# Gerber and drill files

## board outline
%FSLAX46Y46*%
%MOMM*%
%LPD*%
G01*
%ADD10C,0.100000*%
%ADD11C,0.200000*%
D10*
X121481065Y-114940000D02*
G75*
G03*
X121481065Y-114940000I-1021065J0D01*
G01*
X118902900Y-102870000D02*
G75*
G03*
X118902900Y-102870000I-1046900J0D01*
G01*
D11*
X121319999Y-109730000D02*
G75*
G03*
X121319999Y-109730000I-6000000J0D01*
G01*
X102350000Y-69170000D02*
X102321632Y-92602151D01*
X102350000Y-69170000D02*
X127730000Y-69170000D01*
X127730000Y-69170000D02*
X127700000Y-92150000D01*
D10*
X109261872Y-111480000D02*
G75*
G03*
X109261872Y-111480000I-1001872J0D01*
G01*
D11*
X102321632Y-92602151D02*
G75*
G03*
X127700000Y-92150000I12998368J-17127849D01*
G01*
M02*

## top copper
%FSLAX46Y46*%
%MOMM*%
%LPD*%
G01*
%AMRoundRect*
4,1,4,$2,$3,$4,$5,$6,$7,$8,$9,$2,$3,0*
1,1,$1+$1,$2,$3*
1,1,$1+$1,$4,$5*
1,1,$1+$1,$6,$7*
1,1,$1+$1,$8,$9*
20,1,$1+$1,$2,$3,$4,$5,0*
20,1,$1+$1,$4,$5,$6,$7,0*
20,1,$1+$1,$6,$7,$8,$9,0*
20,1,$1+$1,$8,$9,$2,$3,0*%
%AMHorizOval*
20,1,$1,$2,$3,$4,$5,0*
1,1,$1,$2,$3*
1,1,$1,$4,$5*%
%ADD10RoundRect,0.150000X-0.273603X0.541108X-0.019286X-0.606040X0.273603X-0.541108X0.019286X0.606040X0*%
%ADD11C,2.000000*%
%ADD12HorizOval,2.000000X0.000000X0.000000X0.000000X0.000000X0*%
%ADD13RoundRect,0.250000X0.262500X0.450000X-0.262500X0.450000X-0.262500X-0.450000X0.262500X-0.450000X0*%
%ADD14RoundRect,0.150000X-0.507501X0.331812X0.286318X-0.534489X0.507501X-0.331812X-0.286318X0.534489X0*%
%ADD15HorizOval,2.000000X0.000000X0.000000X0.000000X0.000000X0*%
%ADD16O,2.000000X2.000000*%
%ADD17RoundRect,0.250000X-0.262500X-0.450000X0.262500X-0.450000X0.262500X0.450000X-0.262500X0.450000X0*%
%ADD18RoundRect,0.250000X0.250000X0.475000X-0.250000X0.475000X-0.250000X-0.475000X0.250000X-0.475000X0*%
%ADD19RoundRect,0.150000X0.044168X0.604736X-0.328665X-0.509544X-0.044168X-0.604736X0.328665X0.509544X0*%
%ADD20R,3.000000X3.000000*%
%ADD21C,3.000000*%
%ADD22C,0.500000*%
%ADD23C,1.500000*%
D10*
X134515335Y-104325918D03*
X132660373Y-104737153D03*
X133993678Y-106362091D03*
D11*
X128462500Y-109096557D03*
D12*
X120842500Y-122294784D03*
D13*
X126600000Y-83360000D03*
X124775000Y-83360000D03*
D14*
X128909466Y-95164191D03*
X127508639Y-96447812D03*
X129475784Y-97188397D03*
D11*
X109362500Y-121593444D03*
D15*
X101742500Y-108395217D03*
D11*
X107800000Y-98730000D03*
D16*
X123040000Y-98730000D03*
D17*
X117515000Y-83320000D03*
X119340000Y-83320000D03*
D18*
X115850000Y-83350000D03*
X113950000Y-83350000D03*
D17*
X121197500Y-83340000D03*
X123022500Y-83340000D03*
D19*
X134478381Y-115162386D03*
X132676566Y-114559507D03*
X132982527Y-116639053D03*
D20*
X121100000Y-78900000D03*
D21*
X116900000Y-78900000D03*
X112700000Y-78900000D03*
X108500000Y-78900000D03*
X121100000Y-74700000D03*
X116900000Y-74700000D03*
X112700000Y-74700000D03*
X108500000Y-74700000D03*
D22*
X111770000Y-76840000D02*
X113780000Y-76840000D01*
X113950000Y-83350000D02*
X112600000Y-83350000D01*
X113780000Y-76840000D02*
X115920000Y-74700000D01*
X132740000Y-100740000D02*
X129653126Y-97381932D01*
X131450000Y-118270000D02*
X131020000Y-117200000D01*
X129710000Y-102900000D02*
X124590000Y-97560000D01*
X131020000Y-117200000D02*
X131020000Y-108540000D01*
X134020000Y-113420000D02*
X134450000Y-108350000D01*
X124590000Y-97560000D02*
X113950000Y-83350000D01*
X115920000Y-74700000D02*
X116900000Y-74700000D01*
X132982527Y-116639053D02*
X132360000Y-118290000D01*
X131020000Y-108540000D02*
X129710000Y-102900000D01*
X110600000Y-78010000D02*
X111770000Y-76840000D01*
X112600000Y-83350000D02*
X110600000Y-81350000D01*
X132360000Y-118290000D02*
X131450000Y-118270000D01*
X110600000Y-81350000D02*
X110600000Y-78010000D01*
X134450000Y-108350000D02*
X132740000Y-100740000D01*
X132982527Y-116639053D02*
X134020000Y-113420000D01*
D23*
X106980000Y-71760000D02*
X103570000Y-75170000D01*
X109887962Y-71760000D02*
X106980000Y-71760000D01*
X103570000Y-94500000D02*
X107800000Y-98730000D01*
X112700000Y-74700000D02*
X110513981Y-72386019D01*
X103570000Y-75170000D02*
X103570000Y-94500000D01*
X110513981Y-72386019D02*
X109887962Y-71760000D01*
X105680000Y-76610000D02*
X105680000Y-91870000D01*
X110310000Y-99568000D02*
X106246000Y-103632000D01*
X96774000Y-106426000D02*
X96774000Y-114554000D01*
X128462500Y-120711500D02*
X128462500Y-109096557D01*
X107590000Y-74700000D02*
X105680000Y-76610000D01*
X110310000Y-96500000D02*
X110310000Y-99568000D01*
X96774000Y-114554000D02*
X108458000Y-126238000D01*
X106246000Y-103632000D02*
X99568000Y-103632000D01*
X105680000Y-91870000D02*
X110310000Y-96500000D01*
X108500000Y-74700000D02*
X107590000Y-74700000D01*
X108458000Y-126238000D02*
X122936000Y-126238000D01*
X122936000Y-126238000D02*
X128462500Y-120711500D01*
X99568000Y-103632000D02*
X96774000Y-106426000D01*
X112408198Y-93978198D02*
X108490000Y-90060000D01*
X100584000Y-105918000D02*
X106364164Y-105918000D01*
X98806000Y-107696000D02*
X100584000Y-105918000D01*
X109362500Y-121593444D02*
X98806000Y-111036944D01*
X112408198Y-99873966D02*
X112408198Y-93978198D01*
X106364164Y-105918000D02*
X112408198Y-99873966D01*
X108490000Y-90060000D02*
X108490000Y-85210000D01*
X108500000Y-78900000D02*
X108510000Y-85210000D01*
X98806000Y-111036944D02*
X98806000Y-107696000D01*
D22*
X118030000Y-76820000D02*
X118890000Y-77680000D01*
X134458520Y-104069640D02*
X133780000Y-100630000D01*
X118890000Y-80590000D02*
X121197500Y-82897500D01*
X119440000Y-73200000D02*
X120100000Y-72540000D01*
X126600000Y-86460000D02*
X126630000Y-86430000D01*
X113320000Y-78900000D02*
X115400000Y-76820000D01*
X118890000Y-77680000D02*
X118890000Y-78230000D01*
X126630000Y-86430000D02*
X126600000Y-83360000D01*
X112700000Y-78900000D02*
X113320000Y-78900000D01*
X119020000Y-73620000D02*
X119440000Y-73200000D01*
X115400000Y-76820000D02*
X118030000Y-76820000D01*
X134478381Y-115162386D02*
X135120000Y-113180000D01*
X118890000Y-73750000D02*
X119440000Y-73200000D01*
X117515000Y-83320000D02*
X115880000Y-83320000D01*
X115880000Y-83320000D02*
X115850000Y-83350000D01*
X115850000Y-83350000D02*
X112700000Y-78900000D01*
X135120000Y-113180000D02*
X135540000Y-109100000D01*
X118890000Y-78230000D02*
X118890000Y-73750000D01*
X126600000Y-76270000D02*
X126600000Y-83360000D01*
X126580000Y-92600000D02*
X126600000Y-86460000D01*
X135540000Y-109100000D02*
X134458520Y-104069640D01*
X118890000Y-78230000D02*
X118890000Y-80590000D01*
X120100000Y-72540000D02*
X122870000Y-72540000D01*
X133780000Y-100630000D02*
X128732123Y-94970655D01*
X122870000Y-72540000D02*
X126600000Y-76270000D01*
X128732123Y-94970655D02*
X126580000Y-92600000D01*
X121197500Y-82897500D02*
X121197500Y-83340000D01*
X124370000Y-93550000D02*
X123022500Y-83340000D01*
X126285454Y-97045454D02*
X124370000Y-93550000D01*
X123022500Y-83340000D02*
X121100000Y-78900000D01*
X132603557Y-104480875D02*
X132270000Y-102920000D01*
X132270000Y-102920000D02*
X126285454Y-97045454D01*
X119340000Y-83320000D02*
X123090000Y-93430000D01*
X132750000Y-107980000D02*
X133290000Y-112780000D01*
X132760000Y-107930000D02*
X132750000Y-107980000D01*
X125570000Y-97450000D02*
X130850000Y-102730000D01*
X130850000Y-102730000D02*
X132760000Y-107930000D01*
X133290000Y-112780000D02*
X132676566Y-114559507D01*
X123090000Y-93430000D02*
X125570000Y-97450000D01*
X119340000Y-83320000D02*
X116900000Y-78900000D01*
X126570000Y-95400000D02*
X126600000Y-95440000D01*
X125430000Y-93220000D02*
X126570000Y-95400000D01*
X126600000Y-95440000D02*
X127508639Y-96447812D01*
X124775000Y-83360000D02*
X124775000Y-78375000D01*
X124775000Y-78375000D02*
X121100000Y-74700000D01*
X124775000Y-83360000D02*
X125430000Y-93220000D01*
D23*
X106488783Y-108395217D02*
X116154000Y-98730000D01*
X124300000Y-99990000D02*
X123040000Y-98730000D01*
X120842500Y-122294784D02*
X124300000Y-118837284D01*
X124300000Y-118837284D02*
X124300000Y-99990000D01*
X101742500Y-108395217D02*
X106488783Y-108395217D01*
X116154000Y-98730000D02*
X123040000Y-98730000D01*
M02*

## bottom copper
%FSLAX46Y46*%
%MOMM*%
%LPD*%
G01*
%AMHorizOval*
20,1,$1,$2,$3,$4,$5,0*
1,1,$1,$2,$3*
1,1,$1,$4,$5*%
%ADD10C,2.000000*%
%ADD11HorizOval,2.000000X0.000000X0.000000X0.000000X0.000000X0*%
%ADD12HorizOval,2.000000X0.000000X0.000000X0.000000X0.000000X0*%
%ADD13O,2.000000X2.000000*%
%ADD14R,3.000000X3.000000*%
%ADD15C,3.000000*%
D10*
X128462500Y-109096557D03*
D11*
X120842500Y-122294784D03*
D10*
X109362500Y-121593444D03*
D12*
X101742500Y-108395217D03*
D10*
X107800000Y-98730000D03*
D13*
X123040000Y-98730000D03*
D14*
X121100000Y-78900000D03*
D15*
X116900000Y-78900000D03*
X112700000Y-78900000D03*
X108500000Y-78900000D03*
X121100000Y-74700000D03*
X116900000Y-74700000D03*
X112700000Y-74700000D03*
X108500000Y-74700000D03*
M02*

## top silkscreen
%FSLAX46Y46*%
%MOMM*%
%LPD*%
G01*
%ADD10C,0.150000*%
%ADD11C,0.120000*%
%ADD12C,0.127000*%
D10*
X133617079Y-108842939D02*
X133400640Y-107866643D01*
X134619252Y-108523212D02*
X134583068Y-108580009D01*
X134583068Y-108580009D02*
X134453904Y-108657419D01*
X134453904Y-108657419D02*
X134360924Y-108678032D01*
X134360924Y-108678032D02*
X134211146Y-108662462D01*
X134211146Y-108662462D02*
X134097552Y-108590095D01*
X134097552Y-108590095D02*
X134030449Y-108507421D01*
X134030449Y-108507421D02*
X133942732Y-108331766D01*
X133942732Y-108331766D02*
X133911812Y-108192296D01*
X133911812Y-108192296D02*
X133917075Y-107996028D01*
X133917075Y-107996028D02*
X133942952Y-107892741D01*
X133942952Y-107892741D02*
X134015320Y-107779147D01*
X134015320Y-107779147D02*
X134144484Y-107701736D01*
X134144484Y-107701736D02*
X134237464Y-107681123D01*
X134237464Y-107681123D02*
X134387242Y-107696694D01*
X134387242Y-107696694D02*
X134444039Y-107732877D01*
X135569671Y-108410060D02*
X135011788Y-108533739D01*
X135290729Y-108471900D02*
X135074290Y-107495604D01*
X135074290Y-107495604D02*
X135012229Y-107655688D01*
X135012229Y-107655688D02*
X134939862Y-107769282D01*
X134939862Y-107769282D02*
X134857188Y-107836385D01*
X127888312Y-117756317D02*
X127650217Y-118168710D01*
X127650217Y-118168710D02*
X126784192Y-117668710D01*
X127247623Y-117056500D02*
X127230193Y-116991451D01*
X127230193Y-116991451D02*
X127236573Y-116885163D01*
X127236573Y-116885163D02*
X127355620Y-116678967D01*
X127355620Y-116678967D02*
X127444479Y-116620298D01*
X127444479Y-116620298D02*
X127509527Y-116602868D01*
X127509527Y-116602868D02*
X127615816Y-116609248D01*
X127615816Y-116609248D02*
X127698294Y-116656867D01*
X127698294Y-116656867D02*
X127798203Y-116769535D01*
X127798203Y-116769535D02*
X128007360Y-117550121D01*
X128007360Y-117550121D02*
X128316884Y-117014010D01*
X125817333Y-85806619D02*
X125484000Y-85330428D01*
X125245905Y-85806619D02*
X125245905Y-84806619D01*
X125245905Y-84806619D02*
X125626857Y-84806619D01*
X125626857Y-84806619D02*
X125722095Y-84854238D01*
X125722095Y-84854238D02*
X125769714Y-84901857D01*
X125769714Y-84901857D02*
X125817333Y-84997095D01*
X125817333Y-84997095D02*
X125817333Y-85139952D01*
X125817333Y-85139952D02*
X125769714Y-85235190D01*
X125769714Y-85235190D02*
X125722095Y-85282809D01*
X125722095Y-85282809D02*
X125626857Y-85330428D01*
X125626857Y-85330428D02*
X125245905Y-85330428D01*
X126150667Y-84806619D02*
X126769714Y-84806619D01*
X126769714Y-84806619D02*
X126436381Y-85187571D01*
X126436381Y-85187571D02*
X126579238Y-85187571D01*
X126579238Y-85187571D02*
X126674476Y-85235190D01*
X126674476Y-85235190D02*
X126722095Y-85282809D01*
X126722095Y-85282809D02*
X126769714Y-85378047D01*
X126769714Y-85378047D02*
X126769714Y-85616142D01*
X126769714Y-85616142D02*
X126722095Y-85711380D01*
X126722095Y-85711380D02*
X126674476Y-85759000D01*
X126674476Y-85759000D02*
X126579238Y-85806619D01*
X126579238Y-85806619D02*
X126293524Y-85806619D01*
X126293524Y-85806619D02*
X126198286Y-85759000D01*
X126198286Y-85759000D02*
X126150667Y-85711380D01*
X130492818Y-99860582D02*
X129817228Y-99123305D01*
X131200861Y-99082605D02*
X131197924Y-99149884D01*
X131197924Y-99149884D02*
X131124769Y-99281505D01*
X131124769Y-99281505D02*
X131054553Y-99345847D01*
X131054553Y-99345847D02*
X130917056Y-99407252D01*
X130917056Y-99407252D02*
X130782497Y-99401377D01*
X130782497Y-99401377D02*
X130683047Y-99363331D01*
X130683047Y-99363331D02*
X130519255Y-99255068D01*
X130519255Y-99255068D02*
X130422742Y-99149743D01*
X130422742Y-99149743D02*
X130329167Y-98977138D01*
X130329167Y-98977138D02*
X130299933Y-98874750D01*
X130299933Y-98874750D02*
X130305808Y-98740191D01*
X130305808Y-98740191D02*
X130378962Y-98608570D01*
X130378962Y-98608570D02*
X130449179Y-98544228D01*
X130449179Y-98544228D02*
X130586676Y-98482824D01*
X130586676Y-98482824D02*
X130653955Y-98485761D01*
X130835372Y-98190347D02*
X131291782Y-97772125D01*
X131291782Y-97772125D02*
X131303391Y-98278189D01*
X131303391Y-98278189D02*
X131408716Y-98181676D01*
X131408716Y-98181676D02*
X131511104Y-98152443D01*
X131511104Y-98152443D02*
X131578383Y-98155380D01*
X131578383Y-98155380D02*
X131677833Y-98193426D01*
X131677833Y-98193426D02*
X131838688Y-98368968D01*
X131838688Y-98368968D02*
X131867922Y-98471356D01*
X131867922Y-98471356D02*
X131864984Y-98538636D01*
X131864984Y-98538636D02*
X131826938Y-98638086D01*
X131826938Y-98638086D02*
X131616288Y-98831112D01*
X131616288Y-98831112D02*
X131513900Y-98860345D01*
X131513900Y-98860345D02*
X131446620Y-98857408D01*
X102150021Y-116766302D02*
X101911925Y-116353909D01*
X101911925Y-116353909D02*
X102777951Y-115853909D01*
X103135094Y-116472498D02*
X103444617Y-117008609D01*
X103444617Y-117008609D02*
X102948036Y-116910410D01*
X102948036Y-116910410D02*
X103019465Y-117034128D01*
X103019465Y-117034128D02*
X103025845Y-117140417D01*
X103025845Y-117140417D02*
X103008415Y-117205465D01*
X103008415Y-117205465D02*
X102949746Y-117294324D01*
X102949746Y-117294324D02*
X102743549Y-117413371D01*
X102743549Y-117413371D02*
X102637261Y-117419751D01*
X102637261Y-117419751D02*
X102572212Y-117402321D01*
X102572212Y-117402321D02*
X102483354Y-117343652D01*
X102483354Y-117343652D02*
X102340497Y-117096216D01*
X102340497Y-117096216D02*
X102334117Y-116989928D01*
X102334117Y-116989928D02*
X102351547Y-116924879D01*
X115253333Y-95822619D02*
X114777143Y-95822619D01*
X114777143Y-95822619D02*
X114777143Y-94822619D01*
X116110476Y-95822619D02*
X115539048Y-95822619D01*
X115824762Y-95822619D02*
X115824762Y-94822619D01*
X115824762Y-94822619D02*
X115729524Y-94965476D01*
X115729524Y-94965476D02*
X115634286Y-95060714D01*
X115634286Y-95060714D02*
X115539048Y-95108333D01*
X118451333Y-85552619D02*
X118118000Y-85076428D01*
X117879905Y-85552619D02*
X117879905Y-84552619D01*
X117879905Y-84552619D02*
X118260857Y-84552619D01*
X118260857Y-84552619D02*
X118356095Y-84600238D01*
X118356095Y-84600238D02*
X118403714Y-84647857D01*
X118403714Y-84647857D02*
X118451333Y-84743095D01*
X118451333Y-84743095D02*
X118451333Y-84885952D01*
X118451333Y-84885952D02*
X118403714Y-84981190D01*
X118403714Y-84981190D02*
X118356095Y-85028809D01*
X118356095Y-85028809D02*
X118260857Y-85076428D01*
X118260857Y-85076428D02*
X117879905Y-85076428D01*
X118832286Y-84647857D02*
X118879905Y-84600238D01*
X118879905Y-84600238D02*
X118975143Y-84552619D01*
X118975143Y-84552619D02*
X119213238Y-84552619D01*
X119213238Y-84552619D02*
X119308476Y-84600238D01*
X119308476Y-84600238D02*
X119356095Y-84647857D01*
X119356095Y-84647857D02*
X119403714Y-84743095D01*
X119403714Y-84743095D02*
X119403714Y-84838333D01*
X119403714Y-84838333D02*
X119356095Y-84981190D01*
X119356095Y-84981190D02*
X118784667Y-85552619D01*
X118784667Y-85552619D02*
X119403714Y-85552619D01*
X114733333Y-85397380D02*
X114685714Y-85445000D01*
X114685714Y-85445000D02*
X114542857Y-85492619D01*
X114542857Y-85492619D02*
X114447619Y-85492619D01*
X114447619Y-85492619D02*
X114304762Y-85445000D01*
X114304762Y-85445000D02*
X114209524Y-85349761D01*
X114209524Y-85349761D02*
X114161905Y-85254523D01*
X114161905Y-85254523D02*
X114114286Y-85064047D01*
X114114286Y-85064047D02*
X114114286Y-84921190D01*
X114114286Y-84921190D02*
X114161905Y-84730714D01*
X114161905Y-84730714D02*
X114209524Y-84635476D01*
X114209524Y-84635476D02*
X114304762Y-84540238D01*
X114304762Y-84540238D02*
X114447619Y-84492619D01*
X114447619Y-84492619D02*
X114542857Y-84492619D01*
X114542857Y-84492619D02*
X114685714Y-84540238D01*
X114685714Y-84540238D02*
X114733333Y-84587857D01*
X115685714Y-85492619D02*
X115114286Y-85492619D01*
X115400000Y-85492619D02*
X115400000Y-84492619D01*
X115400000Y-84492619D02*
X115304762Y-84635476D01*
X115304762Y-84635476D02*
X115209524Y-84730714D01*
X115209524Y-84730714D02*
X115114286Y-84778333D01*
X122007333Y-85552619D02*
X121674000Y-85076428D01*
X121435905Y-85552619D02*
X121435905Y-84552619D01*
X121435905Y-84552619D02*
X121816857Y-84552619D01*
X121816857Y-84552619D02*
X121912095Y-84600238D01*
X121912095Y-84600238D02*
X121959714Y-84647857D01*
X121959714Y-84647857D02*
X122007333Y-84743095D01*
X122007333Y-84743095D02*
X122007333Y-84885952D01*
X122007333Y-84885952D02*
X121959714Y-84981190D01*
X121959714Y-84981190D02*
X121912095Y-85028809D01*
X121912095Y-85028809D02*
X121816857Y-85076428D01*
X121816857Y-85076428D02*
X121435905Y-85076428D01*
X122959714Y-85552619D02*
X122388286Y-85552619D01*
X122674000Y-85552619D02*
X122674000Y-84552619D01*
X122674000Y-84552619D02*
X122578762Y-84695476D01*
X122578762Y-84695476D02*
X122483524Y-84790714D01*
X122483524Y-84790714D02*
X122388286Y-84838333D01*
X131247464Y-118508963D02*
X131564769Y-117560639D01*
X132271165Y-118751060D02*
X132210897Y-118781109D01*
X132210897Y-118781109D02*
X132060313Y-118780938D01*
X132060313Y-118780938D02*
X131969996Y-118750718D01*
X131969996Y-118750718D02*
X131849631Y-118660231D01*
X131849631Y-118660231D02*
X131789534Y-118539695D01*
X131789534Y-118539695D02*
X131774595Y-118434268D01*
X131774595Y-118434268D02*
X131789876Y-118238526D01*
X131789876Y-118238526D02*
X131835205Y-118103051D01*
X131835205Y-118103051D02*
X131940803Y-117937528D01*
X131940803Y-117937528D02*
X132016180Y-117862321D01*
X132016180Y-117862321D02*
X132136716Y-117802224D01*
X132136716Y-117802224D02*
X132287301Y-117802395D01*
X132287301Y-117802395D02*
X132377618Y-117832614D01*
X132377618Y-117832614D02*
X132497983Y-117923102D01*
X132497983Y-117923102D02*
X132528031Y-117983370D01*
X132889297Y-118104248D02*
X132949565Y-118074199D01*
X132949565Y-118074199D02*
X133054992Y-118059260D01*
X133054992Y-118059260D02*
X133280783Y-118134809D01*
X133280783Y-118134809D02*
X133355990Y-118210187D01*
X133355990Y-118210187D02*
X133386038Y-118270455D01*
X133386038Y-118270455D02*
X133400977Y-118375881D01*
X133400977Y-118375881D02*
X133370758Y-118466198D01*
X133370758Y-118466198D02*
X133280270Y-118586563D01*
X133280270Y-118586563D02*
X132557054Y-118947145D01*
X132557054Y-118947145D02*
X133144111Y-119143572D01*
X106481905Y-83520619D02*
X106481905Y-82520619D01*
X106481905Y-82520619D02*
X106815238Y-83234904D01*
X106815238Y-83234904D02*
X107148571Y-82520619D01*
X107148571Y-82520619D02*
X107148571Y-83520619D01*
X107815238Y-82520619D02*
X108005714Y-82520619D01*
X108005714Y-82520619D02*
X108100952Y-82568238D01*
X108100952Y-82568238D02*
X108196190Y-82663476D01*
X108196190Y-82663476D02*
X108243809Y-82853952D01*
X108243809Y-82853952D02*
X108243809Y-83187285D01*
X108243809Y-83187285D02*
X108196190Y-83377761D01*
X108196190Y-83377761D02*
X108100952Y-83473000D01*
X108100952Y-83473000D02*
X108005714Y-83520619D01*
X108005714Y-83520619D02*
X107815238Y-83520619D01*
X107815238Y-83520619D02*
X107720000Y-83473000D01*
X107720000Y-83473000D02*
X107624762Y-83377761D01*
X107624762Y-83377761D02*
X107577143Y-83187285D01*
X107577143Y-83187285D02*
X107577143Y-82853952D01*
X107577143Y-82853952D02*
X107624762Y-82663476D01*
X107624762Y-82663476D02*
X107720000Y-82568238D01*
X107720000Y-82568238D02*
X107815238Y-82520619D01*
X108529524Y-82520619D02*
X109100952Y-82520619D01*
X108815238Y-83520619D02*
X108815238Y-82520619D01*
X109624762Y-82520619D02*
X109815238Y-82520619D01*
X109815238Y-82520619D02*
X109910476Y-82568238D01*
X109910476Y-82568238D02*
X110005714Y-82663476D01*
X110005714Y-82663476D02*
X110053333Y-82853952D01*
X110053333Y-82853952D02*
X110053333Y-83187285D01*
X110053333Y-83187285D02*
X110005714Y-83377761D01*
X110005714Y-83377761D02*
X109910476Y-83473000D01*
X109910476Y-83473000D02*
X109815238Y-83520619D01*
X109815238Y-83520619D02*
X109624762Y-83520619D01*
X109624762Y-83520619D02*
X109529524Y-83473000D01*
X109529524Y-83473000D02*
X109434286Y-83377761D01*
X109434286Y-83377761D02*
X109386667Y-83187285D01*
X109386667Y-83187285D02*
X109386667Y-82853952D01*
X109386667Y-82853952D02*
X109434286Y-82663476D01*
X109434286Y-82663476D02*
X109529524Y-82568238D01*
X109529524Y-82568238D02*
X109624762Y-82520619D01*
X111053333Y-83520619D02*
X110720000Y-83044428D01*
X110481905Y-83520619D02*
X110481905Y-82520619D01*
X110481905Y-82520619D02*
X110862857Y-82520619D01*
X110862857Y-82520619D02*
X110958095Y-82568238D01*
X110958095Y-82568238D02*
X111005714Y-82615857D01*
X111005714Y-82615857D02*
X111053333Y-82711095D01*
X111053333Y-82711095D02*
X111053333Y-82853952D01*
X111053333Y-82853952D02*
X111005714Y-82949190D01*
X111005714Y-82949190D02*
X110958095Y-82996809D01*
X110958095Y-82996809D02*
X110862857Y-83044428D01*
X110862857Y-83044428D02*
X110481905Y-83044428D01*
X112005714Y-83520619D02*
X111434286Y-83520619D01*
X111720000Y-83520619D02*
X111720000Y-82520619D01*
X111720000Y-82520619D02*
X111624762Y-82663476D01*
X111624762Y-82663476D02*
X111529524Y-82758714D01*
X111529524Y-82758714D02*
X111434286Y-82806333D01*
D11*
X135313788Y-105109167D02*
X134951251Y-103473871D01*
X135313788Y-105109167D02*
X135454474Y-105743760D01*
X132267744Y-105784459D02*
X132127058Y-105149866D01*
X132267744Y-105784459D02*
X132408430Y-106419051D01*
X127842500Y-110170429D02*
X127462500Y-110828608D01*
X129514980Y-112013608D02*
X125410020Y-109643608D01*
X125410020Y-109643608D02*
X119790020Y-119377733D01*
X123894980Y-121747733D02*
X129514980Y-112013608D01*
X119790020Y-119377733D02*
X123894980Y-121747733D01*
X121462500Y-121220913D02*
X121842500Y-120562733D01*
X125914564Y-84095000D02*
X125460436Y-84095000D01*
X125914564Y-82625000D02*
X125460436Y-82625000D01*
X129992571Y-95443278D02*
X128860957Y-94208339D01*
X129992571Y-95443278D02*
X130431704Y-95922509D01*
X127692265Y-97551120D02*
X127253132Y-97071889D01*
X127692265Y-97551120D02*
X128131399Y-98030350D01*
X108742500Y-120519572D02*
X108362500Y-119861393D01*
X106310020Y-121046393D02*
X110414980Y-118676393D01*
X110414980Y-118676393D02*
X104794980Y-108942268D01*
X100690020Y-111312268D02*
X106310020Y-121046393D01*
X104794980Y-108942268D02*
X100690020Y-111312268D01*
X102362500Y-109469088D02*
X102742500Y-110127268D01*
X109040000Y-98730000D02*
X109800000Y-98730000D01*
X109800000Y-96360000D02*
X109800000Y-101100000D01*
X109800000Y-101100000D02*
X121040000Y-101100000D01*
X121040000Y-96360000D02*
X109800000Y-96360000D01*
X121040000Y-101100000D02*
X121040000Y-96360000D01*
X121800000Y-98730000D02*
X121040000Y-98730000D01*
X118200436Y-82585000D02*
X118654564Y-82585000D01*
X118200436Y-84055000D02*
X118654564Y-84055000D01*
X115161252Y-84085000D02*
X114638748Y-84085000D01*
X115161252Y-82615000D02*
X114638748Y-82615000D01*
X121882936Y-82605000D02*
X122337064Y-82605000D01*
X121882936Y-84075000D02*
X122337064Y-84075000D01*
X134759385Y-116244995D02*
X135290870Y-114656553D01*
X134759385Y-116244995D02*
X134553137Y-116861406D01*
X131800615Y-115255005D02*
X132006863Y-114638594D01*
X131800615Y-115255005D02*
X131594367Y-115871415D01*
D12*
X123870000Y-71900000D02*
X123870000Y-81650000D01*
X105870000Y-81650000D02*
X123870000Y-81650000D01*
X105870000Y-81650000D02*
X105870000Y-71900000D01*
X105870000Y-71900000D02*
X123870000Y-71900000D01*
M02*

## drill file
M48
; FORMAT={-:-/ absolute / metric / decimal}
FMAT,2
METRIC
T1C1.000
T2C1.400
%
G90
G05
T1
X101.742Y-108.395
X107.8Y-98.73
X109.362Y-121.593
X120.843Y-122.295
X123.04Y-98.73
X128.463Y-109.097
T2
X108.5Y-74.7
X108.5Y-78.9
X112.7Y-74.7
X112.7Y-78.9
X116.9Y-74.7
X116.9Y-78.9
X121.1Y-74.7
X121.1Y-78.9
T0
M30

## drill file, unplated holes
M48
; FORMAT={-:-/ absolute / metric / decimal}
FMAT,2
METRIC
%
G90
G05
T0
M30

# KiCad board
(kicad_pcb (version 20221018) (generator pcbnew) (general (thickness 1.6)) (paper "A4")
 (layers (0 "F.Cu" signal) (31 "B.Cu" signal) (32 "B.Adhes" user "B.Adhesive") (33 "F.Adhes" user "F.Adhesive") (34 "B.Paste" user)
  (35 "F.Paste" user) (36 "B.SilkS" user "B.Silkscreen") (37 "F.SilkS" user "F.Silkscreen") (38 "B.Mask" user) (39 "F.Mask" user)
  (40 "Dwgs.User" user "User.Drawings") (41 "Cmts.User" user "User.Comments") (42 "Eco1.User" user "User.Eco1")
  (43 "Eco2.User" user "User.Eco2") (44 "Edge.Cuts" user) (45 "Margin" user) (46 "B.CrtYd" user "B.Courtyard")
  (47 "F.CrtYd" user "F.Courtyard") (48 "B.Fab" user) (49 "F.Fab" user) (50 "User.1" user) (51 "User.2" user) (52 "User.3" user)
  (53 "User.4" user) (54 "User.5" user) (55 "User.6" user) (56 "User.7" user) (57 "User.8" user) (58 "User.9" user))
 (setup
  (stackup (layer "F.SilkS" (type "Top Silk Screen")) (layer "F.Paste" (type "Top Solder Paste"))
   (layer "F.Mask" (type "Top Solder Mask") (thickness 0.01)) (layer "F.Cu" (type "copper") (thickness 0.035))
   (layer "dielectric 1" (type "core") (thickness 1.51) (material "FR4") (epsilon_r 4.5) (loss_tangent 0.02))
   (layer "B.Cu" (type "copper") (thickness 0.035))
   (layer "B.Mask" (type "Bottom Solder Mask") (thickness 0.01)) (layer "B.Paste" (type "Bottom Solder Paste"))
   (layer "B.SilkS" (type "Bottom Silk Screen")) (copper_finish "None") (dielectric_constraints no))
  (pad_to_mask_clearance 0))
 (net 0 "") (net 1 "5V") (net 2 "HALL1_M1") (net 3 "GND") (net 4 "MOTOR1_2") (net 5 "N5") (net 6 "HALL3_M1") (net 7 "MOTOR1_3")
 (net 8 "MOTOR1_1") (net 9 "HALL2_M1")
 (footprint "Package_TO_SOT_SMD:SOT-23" (layer "F.Cu") (at 133.790766 105.446813 -77.5)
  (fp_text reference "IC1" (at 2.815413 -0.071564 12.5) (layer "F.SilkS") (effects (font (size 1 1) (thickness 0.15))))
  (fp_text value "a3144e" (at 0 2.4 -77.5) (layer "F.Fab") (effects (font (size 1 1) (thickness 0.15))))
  (fp_line (start 0 -1.56) (end -1.675 -1.56) (stroke (width 0.12) (type solid)) (layer "F.SilkS"))
  (fp_line (start 0 -1.56) (end 0.65 -1.56) (stroke (width 0.12) (type solid)) (layer "F.SilkS"))
  (fp_line (start 0 1.56) (end -0.65 1.56) (stroke (width 0.12) (type solid)) (layer "F.SilkS"))
  (fp_line (start 0 1.56) (end 0.65 1.56) (stroke (width 0.12) (type solid)) (layer "F.SilkS"))
  (pad "1" smd roundrect (at -0.9375 -0.95 282.5) (size 1.475 0.6) (layers "F.Cu" "F.Paste" "F.Mask") (roundrect_rratio 0.25) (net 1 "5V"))
  (pad "2" smd roundrect (at -0.9375 0.95 282.5) (size 1.475 0.6) (layers "F.Cu" "F.Paste" "F.Mask") (roundrect_rratio 0.25)
   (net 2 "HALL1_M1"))
  (pad "3" smd roundrect (at 0.9375 0 282.5) (size 1.475 0.6) (layers "F.Cu" "F.Paste" "F.Mask") (roundrect_rratio 0.25) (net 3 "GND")))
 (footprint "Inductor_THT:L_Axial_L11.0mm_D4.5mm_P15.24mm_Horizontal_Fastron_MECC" (layer "F.Cu") (at 128.4625 109.096557 -120)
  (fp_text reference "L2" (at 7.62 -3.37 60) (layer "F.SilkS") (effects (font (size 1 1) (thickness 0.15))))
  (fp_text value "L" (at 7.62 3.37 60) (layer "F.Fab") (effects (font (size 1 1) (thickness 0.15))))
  (fp_line (start 1.24 0) (end 2 0) (stroke (width 0.12) (type solid)) (layer "F.SilkS"))
  (fp_line (start 2 -2.37) (end 2 2.37) (stroke (width 0.12) (type solid)) (layer "F.SilkS"))
  (fp_line (start 2 2.37) (end 13.24 2.37) (stroke (width 0.12) (type solid)) (layer "F.SilkS"))
  (fp_line (start 13.24 -2.37) (end 2 -2.37) (stroke (width 0.12) (type solid)) (layer "F.SilkS"))
  (fp_line (start 13.24 2.37) (end 13.24 -2.37) (stroke (width 0.12) (type solid)) (layer "F.SilkS"))
  (fp_line (start 14 0) (end 13.24 0) (stroke (width 0.12) (type solid)) (layer "F.SilkS"))
  (pad "1" thru_hole circle (at 0 0 240) (size 2 2) (drill 1) (layers "*.Cu" "*.Mask") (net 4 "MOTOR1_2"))
  (pad "2" thru_hole oval (at 15.24 0 240) (size 2 2) (drill 1) (layers "*.Cu" "*.Mask") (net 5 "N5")))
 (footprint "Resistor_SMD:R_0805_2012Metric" (layer "F.Cu") (at 125.6875 83.36 180)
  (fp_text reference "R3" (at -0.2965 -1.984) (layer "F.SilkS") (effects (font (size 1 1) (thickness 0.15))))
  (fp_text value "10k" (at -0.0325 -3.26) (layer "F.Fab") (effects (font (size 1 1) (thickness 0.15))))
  (fp_line (start -0.227064 -0.735) (end 0.227064 -0.735) (stroke (width 0.12) (type solid)) (layer "F.SilkS"))
  (fp_line (start -0.227064 0.735) (end 0.227064 0.735) (stroke (width 0.12) (type solid)) (layer "F.SilkS"))
  (pad "1" smd roundrect (at -0.9125 0 180) (size 1.025 1.4) (layers "F.Cu" "F.Paste" "F.Mask") (roundrect_rratio 0.243902439) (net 1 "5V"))
  (pad "2" smd roundrect (at 0.9125 0 180) (size 1.025 1.4) (layers "F.Cu" "F.Paste" "F.Mask") (roundrect_rratio 0.243902439)
   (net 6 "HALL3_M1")))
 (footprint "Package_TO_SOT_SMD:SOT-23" (layer "F.Cu") (at 128.842418 96.497199 -47.5)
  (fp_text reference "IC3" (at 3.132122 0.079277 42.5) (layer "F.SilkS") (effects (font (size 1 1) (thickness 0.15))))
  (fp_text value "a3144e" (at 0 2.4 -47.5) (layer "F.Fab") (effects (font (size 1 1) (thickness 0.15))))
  (fp_line (start 0 -1.56) (end -1.675 -1.56) (stroke (width 0.12) (type solid)) (layer "F.SilkS"))
  (fp_line (start 0 -1.56) (end 0.65 -1.56) (stroke (width 0.12) (type solid)) (layer "F.SilkS"))
  (fp_line (start 0 1.56) (end -0.65 1.56) (stroke (width 0.12) (type solid)) (layer "F.SilkS"))
  (fp_line (start 0 1.56) (end 0.65 1.56) (stroke (width 0.12) (type solid)) (layer "F.SilkS"))
  (pad "1" smd roundrect (at -0.9375 -0.95 312.5) (size 1.475 0.6) (layers "F.Cu" "F.Paste" "F.Mask") (roundrect_rratio 0.25) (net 1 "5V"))
  (pad "2" smd roundrect (at -0.9375 0.95 312.5) (size 1.475 0.6) (layers "F.Cu" "F.Paste" "F.Mask") (roundrect_rratio 0.25)
   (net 6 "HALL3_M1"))
  (pad "3" smd roundrect (at 0.9375 0 312.5) (size 1.475 0.6) (layers "F.Cu" "F.Paste" "F.Mask") (roundrect_rratio 0.25) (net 3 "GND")))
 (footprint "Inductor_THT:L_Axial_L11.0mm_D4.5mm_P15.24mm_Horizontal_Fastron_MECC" (layer "F.Cu") (at 109.3625 121.593444 120)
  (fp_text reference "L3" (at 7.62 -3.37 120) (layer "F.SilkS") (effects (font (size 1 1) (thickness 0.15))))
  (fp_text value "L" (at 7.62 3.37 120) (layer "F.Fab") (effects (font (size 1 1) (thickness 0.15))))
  (fp_line (start 1.24 0) (end 2 0) (stroke (width 0.12) (type solid)) (layer "F.SilkS"))
  (fp_line (start 2 -2.37) (end 2 2.37) (stroke (width 0.12) (type solid)) (layer "F.SilkS"))
  (fp_line (start 2 2.37) (end 13.24 2.37) (stroke (width 0.12) (type solid)) (layer "F.SilkS"))
  (fp_line (start 13.24 -2.37) (end 2 -2.37) (stroke (width 0.12) (type solid)) (layer "F.SilkS"))
  (fp_line (start 13.24 2.37) (end 13.24 -2.37) (stroke (width 0.12) (type solid)) (layer "F.SilkS"))
  (fp_line (start 14 0) (end 13.24 0) (stroke (width 0.12) (type solid)) (layer "F.SilkS"))
  (pad "1" thru_hole circle (at 0 0 120) (size 2 2) (drill 1) (layers "*.Cu" "*.Mask") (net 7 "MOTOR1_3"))
  (pad "2" thru_hole oval (at 15.24 0 120) (size 2 2) (drill 1) (layers "*.Cu" "*.Mask") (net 5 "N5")))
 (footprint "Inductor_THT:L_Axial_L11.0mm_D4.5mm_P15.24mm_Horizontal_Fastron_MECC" (layer "F.Cu") (at 107.8 98.73)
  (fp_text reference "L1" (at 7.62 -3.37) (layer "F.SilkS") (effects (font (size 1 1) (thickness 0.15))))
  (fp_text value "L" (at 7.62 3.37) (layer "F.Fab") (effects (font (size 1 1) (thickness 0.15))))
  (fp_line (start 1.24 0) (end 2 0) (stroke (width 0.12) (type solid)) (layer "F.SilkS"))
  (fp_line (start 2 -2.37) (end 2 2.37) (stroke (width 0.12) (type solid)) (layer "F.SilkS"))
  (fp_line (start 2 2.37) (end 13.24 2.37) (stroke (width 0.12) (type solid)) (layer "F.SilkS"))
  (fp_line (start 13.24 -2.37) (end 2 -2.37) (stroke (width 0.12) (type solid)) (layer "F.SilkS"))
  (fp_line (start 13.24 2.37) (end 13.24 -2.37) (stroke (width 0.12) (type solid)) (layer "F.SilkS"))
  (fp_line (start 14 0) (end 13.24 0) (stroke (width 0.12) (type solid)) (layer "F.SilkS"))
  (pad "1" thru_hole circle (at 0 0) (size 2 2) (drill 1) (layers "*.Cu" "*.Mask") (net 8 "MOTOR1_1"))
  (pad "2" thru_hole oval (at 15.24 0) (size 2 2) (drill 1) (layers "*.Cu" "*.Mask") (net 5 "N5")))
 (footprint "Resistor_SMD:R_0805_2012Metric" (layer "F.Cu") (at 118.4275 83.32)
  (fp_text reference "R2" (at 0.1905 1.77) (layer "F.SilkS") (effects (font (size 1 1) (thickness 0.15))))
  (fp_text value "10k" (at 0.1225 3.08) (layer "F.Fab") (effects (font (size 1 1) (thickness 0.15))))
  (fp_line (start -0.227064 -0.735) (end 0.227064 -0.735) (stroke (width 0.12) (type solid)) (layer "F.SilkS"))
  (fp_line (start -0.227064 0.735) (end 0.227064 0.735) (stroke (width 0.12) (type solid)) (layer "F.SilkS"))
  (pad "1" smd roundrect (at -0.9125 0) (size 1.025 1.4) (layers "F.Cu" "F.Paste" "F.Mask") (roundrect_rratio 0.243902439) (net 1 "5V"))
  (pad "2" smd roundrect (at 0.9125 0) (size 1.025 1.4) (layers "F.Cu" "F.Paste" "F.Mask") (roundrect_rratio 0.243902439) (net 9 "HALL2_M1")))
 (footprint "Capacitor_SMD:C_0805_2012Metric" (layer "F.Cu") (at 114.9 83.35 180)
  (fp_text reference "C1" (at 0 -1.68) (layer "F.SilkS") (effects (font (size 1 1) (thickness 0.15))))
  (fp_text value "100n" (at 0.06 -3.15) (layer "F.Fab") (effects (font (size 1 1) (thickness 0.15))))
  (fp_line (start -0.261252 -0.735) (end 0.261252 -0.735) (stroke (width 0.12) (type solid)) (layer "F.SilkS"))
  (fp_line (start -0.261252 0.735) (end 0.261252 0.735) (stroke (width 0.12) (type solid)) (layer "F.SilkS"))
  (pad "1" smd roundrect (at -0.95 0 180) (size 1 1.45) (layers "F.Cu" "F.Paste" "F.Mask") (roundrect_rratio 0.25) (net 1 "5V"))
  (pad "2" smd roundrect (at 0.95 0 180) (size 1 1.45) (layers "F.Cu" "F.Paste" "F.Mask") (roundrect_rratio 0.25) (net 3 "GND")))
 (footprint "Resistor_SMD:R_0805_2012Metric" (layer "F.Cu") (at 122.11 83.34)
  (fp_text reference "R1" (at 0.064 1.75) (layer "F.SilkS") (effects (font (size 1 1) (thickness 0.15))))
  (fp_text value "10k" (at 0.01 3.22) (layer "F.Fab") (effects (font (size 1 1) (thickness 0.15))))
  (fp_line (start -0.227064 -0.735) (end 0.227064 -0.735) (stroke (width 0.12) (type solid)) (layer "F.SilkS"))
  (fp_line (start -0.227064 0.735) (end 0.227064 0.735) (stroke (width 0.12) (type solid)) (layer "F.SilkS"))
  (pad "1" smd roundrect (at -0.9125 0) (size 1.025 1.4) (layers "F.Cu" "F.Paste" "F.Mask") (roundrect_rratio 0.243902439) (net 1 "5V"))
  (pad "2" smd roundrect (at 0.9125 0) (size 1.025 1.4) (layers "F.Cu" "F.Paste" "F.Mask") (roundrect_rratio 0.243902439) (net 2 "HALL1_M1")))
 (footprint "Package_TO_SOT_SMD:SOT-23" (layer "F.Cu") (at 133.28 115.75 -108.5)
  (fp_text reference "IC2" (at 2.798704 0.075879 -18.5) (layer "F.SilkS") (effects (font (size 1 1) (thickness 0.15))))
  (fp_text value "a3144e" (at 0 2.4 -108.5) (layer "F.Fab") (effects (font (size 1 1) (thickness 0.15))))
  (fp_line (start 0 -1.56) (end -1.675 -1.56) (stroke (width 0.12) (type solid)) (layer "F.SilkS"))
  (fp_line (start 0 -1.56) (end 0.65 -1.56) (stroke (width 0.12) (type solid)) (layer "F.SilkS"))
  (fp_line (start 0 1.56) (end -0.65 1.56) (stroke (width 0.12) (type solid)) (layer "F.SilkS"))
  (fp_line (start 0 1.56) (end 0.65 1.56) (stroke (width 0.12) (type solid)) (layer "F.SilkS"))
  (pad "1" smd roundrect (at -0.9375 -0.95 251.5) (size 1.475 0.6) (layers "F.Cu" "F.Paste" "F.Mask") (roundrect_rratio 0.25) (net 1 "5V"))
  (pad "2" smd roundrect (at -0.9375 0.95 251.5) (size 1.475 0.6) (layers "F.Cu" "F.Paste" "F.Mask") (roundrect_rratio 0.25)
   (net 9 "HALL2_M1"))
  (pad "3" smd roundrect (at 0.9375 0 251.5) (size 1.475 0.6) (layers "F.Cu" "F.Paste" "F.Mask") (roundrect_rratio 0.25) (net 3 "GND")))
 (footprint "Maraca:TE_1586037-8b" (layer "F.Cu") (at 121.1 78.9 180)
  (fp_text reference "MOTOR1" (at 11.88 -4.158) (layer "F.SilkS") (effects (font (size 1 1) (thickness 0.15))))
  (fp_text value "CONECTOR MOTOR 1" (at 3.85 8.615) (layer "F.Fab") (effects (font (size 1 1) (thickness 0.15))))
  (fp_line (start -2.77 7) (end -2.77 -2.75) (stroke (width 0.127) (type solid)) (layer "F.SilkS"))
  (fp_line (start 15.23 -2.75) (end -2.77 -2.75) (stroke (width 0.127) (type solid)) (layer "F.SilkS"))
  (fp_line (start 15.23 -2.75) (end 15.23 7) (stroke (width 0.127) (type solid)) (layer "F.SilkS"))
  (fp_line (start 15.23 7) (end -2.77 7) (stroke (width 0.127) (type solid)) (layer "F.SilkS"))
  (pad "1" thru_hole rect (at 0 0 180) (size 3 3) (drill 1.4) (layers "*.Cu" "*.Mask") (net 2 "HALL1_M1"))
  (pad "2" thru_hole circle (at 4.2 0 180) (size 3 3) (drill 1.4) (layers "*.Cu" "*.Mask") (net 9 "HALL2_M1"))
  (pad "3" thru_hole circle (at 8.4 0 180) (size 3 3) (drill 1.4) (layers "*.Cu" "*.Mask") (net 1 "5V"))
  (pad "4" thru_hole circle (at 12.6 0 180) (size 3 3) (drill 1.4) (layers "*.Cu" "*.Mask") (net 7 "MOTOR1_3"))
  (pad "5" thru_hole circle (at 0 4.2 180) (size 3 3) (drill 1.4) (layers "*.Cu" "*.Mask") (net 6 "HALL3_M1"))
  (pad "6" thru_hole circle (at 4.2 4.2 180) (size 3 3) (drill 1.4) (layers "*.Cu" "*.Mask") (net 3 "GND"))
  (pad "7" thru_hole circle (at 8.4 4.2 180) (size 3 3) (drill 1.4) (layers "*.Cu" "*.Mask") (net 8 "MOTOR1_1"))
  (pad "8" thru_hole circle (at 12.6 4.2 180) (size 3 3) (drill 1.4) (layers "*.Cu" "*.Mask") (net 4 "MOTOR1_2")))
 (gr_circle (center 120.46 114.94) (end 121.481065 114.94) (stroke (width 0.1) (type default)) (fill none) (layer "Edge.Cuts"))
 (gr_circle (center 117.856 102.87) (end 118.896 102.99) (stroke (width 0.1) (type default)) (fill none) (layer "Edge.Cuts"))
 (gr_circle (center 115.319999 109.73) (end 121.319999 109.73) (stroke (width 0.2) (type default)) (fill none) (layer "Edge.Cuts"))
 (gr_line (start 102.35 69.17) (end 102.321632 92.602151) (stroke (width 0.2) (type default)) (layer "Edge.Cuts"))
 (gr_line (start 102.35 69.17) (end 127.73 69.17) (stroke (width 0.2) (type default)) (layer "Edge.Cuts"))
 (gr_line (start 127.73 69.17) (end 127.7 92.15) (stroke (width 0.2) (type default)) (layer "Edge.Cuts"))
 (gr_circle (center 108.26 111.48) (end 109.260624 111.43) (stroke (width 0.1) (type default)) (fill none) (layer "Edge.Cuts"))
 (gr_arc (start 127.7 92.15) (mid 115.703019 131.228235) (end 102.321632 92.602151) (stroke (width 0.2) (type default)) (layer "Edge.Cuts"))
 (segment (start 111.77 76.84) (end 113.78 76.84) (width 0.5) (layer "F.Cu") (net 3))
 (segment (start 113.95 83.35) (end 112.6 83.35) (width 0.5) (layer "F.Cu") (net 3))
 (segment (start 113.78 76.84) (end 115.92 74.7) (width 0.5) (layer "F.Cu") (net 3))
 (segment (start 132.74 100.74) (end 129.653126 97.381932) (width 0.5) (layer "F.Cu") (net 3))
 (segment (start 131.45 118.27) (end 131.02 117.2) (width 0.5) (layer "F.Cu") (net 3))
 (segment (start 129.71 102.9) (end 124.59 97.56) (width 0.5) (layer "F.Cu") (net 3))
 (segment (start 131.02 117.2) (end 131.02 108.54) (width 0.5) (layer "F.Cu") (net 3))
 (segment (start 134.02 113.42) (end 134.45 108.35) (width 0.5) (layer "F.Cu") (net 3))
 (segment (start 124.59 97.56) (end 113.95 83.35) (width 0.5) (layer "F.Cu") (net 3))
 (segment (start 115.92 74.7) (end 116.9 74.7) (width 0.5) (layer "F.Cu") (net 3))
 (segment (start 132.982527 116.639053) (end 132.36 118.29) (width 0.5) (layer "F.Cu") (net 3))
 (segment (start 131.02 108.54) (end 129.71 102.9) (width 0.5) (layer "F.Cu") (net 3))
 (segment (start 110.6 78.01) (end 111.77 76.84) (width 0.5) (layer "F.Cu") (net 3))
 (segment (start 112.6 83.35) (end 110.6 81.35) (width 0.5) (layer "F.Cu") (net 3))
 (segment (start 132.36 118.29) (end 131.45 118.27) (width 0.5) (layer "F.Cu") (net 3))
 (segment (start 110.6 81.35) (end 110.6 78.01) (width 0.5) (layer "F.Cu") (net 3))
 (segment (start 134.45 108.35) (end 132.74 100.74) (width 0.5) (layer "F.Cu") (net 3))
 (segment (start 132.982527 116.639053) (end 134.02 113.42) (width 0.5) (layer "F.Cu") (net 3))
 (segment (start 106.98 71.76) (end 103.57 75.17) (width 1.5) (layer "F.Cu") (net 8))
 (segment (start 109.887962 71.76) (end 106.98 71.76) (width 1.5) (layer "F.Cu") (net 8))
 (segment (start 103.57 94.5) (end 107.8 98.73) (width 1.5) (layer "F.Cu") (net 8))
 (segment (start 112.7 74.7) (end 110.513981 72.386019) (width 1.5) (layer "F.Cu") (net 8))
 (segment (start 103.57 75.17) (end 103.57 94.5) (width 1.5) (layer "F.Cu") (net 8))
 (segment (start 110.513981 72.386019) (end 109.887962 71.76) (width 1.5) (layer "F.Cu") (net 8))
 (segment (start 105.68 76.61) (end 105.68 91.87) (width 1.5) (layer "F.Cu") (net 4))
 (segment (start 110.31 99.568) (end 106.246 103.632) (width 1.5) (layer "F.Cu") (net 4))
 (segment (start 96.774 106.426) (end 96.774 114.554) (width 1.5) (layer "F.Cu") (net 4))
 (segment (start 128.4625 120.7115) (end 128.4625 109.096557) (width 1.5) (layer "F.Cu") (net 4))
 (segment (start 107.59 74.7) (end 105.68 76.61) (width 1.5) (layer "F.Cu") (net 4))
 (segment (start 110.31 96.5) (end 110.31 99.568) (width 1.5) (layer "F.Cu") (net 4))
 (segment (start 96.774 114.554) (end 108.458 126.238) (width 1.5) (layer "F.Cu") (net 4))
 (segment (start 106.246 103.632) (end 99.568 103.632) (width 1.5) (layer "F.Cu") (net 4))
 (segment (start 105.68 91.87) (end 110.31 96.5) (width 1.5) (layer "F.Cu") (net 4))
 (segment (start 108.5 74.7) (end 107.59 74.7) (width 1.5) (layer "F.Cu") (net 4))
 (segment (start 108.458 126.238) (end 122.936 126.238) (width 1.5) (layer "F.Cu") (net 4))
 (segment (start 122.936 126.238) (end 128.4625 120.7115) (width 1.5) (layer "F.Cu") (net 4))
 (segment (start 99.568 103.632) (end 96.774 106.426) (width 1.5) (layer "F.Cu") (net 4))
 (segment (start 112.408198 93.978198) (end 108.49 90.06) (width 1.5) (layer "F.Cu") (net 7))
 (segment (start 100.584 105.918) (end 106.364164 105.918) (width 1.5) (layer "F.Cu") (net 7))
 (segment (start 98.806 107.696) (end 100.584 105.918) (width 1.5) (layer "F.Cu") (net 7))
 (segment (start 109.3625 121.593444) (end 98.806 111.036944) (width 1.5) (layer "F.Cu") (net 7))
 (segment (start 112.408198 99.873966) (end 112.408198 93.978198) (width 1.5) (layer "F.Cu") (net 7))
 (segment (start 106.364164 105.918) (end 112.408198 99.873966) (width 1.5) (layer "F.Cu") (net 7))
 (segment (start 108.49 90.06) (end 108.49 85.21) (width 1.5) (layer "F.Cu") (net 7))
 (segment (start 108.5 78.9) (end 108.51 85.21) (width 1.5) (layer "F.Cu") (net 7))
 (segment (start 98.806 111.036944) (end 98.806 107.696) (width 1.5) (layer "F.Cu") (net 7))
 (segment (start 118.03 76.82) (end 118.89 77.68) (width 0.5) (layer "F.Cu") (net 1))
 (segment (start 134.45852 104.06964) (end 133.78 100.63) (width 0.5) (layer "F.Cu") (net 1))
 (segment (start 118.89 80.59) (end 121.1975 82.8975) (width 0.5) (layer "F.Cu") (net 1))
 (segment (start 119.44 73.2) (end 120.1 72.54) (width 0.5) (layer "F.Cu") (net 1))
 (segment (start 126.6 86.46) (end 126.63 86.43) (width 0.5) (layer "F.Cu") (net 1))
 (segment (start 113.32 78.9) (end 115.4 76.82) (width 0.5) (layer "F.Cu") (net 1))
 (segment (start 118.89 77.68) (end 118.89 78.23) (width 0.5) (layer "F.Cu") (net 1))
 (segment (start 126.63 86.43) (end 126.6 83.36) (width 0.5) (layer "F.Cu") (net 1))
 (segment (start 112.7 78.9) (end 113.32 78.9) (width 0.5) (layer "F.Cu") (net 1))
 (segment (start 119.02 73.62) (end 119.44 73.2) (width 0.5) (layer "F.Cu") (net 1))
 (segment (start 115.4 76.82) (end 118.03 76.82) (width 0.5) (layer "F.Cu") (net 1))
 (segment (start 134.478381 115.162386) (end 135.12 113.18) (width 0.5) (layer "F.Cu") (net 1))
 (segment (start 118.89 73.75) (end 119.44 73.2) (width 0.5) (layer "F.Cu") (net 1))
 (segment (start 117.515 83.32) (end 115.88 83.32) (width 0.5) (layer "F.Cu") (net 1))
 (segment (start 115.88 83.32) (end 115.85 83.35) (width 0.5) (layer "F.Cu") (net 1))
 (segment (start 115.85 83.35) (end 112.7 78.9) (width 0.5) (layer "F.Cu") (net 1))
 (segment (start 135.12 113.18) (end 135.54 109.1) (width 0.5) (layer "F.Cu") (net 1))
 (segment (start 118.89 78.23) (end 118.89 73.75) (width 0.5) (layer "F.Cu") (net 1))
 (segment (start 126.6 76.27) (end 126.6 83.36) (width 0.5) (layer "F.Cu") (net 1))
 (segment (start 126.58 92.6) (end 126.6 86.46) (width 0.5) (layer "F.Cu") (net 1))
 (segment (start 135.54 109.1) (end 134.45852 104.06964) (width 0.5) (layer "F.Cu") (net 1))
 (segment (start 118.89 78.23) (end 118.89 80.59) (width 0.5) (layer "F.Cu") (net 1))
 (segment (start 120.1 72.54) (end 122.87 72.54) (width 0.5) (layer "F.Cu") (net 1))
 (segment (start 133.78 100.63) (end 128.732123 94.970655) (width 0.5) (layer "F.Cu") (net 1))
 (segment (start 122.87 72.54) (end 126.6 76.27) (width 0.5) (layer "F.Cu") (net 1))
 (segment (start 128.732123 94.970655) (end 126.58 92.6) (width 0.5) (layer "F.Cu") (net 1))
 (segment (start 121.1975 82.8975) (end 121.1975 83.34) (width 0.5) (layer "F.Cu") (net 1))
 (segment (start 124.37 93.55) (end 123.0225 83.34) (width 0.5) (layer "F.Cu") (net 2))
 (segment (start 126.285454 97.045454) (end 124.37 93.55) (width 0.5) (layer "F.Cu") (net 2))
 (segment (start 123.0225 83.34) (end 121.1 78.9) (width 0.5) (layer "F.Cu") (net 2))
 (segment (start 132.603557 104.480875) (end 132.27 102.92) (width 0.5) (layer "F.Cu") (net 2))
 (segment (start 132.27 102.92) (end 126.285454 97.045454) (width 0.5) (layer "F.Cu") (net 2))
 (segment (start 119.34 83.32) (end 123.09 93.43) (width 0.5) (layer "F.Cu") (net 9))
 (segment (start 132.75 107.98) (end 133.29 112.78) (width 0.5) (layer "F.Cu") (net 9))
 (segment (start 132.76 107.93) (end 132.75 107.98) (width 0.5) (layer "F.Cu") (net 9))
 (segment (start 125.57 97.45) (end 130.85 102.73) (width 0.5) (layer "F.Cu") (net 9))
 (segment (start 130.85 102.73) (end 132.76 107.93) (width 0.5) (layer "F.Cu") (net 9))
 (segment (start 133.29 112.78) (end 132.676566 114.559507) (width 0.5) (layer "F.Cu") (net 9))
 (segment (start 123.09 93.43) (end 125.57 97.45) (width 0.5) (layer "F.Cu") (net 9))
 (segment (start 119.34 83.32) (end 116.9 78.9) (width 0.5) (layer "F.Cu") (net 9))
 (segment (start 126.57 95.4) (end 126.6 95.44) (width 0.5) (layer "F.Cu") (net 6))
 (segment (start 125.43 93.22) (end 126.57 95.4) (width 0.5) (layer "F.Cu") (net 6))
 (segment (start 126.6 95.44) (end 127.508639 96.447812) (width 0.5) (layer "F.Cu") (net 6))
 (segment (start 124.775 83.36) (end 124.775 78.375) (width 0.5) (layer "F.Cu") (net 6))
 (segment (start 124.775 78.375) (end 121.1 74.7) (width 0.5) (layer "F.Cu") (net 6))
 (segment (start 124.775 83.36) (end 125.43 93.22) (width 0.5) (layer "F.Cu") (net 6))
 (segment (start 106.488783 108.395217) (end 116.154 98.73) (width 1.5) (layer "F.Cu") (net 5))
 (segment (start 124.3 99.99) (end 123.04 98.73) (width 1.5) (layer "F.Cu") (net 5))
 (segment (start 120.8425 122.294784) (end 124.3 118.837284) (width 1.5) (layer "F.Cu") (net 5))
 (segment (start 124.3 118.837284) (end 124.3 99.99) (width 1.5) (layer "F.Cu") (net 5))
 (segment (start 101.7425 108.395217) (end 106.488783 108.395217) (width 1.5) (layer "F.Cu") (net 5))
 (segment (start 116.154 98.73) (end 123.04 98.73) (width 1.5) (layer "F.Cu") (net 5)))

